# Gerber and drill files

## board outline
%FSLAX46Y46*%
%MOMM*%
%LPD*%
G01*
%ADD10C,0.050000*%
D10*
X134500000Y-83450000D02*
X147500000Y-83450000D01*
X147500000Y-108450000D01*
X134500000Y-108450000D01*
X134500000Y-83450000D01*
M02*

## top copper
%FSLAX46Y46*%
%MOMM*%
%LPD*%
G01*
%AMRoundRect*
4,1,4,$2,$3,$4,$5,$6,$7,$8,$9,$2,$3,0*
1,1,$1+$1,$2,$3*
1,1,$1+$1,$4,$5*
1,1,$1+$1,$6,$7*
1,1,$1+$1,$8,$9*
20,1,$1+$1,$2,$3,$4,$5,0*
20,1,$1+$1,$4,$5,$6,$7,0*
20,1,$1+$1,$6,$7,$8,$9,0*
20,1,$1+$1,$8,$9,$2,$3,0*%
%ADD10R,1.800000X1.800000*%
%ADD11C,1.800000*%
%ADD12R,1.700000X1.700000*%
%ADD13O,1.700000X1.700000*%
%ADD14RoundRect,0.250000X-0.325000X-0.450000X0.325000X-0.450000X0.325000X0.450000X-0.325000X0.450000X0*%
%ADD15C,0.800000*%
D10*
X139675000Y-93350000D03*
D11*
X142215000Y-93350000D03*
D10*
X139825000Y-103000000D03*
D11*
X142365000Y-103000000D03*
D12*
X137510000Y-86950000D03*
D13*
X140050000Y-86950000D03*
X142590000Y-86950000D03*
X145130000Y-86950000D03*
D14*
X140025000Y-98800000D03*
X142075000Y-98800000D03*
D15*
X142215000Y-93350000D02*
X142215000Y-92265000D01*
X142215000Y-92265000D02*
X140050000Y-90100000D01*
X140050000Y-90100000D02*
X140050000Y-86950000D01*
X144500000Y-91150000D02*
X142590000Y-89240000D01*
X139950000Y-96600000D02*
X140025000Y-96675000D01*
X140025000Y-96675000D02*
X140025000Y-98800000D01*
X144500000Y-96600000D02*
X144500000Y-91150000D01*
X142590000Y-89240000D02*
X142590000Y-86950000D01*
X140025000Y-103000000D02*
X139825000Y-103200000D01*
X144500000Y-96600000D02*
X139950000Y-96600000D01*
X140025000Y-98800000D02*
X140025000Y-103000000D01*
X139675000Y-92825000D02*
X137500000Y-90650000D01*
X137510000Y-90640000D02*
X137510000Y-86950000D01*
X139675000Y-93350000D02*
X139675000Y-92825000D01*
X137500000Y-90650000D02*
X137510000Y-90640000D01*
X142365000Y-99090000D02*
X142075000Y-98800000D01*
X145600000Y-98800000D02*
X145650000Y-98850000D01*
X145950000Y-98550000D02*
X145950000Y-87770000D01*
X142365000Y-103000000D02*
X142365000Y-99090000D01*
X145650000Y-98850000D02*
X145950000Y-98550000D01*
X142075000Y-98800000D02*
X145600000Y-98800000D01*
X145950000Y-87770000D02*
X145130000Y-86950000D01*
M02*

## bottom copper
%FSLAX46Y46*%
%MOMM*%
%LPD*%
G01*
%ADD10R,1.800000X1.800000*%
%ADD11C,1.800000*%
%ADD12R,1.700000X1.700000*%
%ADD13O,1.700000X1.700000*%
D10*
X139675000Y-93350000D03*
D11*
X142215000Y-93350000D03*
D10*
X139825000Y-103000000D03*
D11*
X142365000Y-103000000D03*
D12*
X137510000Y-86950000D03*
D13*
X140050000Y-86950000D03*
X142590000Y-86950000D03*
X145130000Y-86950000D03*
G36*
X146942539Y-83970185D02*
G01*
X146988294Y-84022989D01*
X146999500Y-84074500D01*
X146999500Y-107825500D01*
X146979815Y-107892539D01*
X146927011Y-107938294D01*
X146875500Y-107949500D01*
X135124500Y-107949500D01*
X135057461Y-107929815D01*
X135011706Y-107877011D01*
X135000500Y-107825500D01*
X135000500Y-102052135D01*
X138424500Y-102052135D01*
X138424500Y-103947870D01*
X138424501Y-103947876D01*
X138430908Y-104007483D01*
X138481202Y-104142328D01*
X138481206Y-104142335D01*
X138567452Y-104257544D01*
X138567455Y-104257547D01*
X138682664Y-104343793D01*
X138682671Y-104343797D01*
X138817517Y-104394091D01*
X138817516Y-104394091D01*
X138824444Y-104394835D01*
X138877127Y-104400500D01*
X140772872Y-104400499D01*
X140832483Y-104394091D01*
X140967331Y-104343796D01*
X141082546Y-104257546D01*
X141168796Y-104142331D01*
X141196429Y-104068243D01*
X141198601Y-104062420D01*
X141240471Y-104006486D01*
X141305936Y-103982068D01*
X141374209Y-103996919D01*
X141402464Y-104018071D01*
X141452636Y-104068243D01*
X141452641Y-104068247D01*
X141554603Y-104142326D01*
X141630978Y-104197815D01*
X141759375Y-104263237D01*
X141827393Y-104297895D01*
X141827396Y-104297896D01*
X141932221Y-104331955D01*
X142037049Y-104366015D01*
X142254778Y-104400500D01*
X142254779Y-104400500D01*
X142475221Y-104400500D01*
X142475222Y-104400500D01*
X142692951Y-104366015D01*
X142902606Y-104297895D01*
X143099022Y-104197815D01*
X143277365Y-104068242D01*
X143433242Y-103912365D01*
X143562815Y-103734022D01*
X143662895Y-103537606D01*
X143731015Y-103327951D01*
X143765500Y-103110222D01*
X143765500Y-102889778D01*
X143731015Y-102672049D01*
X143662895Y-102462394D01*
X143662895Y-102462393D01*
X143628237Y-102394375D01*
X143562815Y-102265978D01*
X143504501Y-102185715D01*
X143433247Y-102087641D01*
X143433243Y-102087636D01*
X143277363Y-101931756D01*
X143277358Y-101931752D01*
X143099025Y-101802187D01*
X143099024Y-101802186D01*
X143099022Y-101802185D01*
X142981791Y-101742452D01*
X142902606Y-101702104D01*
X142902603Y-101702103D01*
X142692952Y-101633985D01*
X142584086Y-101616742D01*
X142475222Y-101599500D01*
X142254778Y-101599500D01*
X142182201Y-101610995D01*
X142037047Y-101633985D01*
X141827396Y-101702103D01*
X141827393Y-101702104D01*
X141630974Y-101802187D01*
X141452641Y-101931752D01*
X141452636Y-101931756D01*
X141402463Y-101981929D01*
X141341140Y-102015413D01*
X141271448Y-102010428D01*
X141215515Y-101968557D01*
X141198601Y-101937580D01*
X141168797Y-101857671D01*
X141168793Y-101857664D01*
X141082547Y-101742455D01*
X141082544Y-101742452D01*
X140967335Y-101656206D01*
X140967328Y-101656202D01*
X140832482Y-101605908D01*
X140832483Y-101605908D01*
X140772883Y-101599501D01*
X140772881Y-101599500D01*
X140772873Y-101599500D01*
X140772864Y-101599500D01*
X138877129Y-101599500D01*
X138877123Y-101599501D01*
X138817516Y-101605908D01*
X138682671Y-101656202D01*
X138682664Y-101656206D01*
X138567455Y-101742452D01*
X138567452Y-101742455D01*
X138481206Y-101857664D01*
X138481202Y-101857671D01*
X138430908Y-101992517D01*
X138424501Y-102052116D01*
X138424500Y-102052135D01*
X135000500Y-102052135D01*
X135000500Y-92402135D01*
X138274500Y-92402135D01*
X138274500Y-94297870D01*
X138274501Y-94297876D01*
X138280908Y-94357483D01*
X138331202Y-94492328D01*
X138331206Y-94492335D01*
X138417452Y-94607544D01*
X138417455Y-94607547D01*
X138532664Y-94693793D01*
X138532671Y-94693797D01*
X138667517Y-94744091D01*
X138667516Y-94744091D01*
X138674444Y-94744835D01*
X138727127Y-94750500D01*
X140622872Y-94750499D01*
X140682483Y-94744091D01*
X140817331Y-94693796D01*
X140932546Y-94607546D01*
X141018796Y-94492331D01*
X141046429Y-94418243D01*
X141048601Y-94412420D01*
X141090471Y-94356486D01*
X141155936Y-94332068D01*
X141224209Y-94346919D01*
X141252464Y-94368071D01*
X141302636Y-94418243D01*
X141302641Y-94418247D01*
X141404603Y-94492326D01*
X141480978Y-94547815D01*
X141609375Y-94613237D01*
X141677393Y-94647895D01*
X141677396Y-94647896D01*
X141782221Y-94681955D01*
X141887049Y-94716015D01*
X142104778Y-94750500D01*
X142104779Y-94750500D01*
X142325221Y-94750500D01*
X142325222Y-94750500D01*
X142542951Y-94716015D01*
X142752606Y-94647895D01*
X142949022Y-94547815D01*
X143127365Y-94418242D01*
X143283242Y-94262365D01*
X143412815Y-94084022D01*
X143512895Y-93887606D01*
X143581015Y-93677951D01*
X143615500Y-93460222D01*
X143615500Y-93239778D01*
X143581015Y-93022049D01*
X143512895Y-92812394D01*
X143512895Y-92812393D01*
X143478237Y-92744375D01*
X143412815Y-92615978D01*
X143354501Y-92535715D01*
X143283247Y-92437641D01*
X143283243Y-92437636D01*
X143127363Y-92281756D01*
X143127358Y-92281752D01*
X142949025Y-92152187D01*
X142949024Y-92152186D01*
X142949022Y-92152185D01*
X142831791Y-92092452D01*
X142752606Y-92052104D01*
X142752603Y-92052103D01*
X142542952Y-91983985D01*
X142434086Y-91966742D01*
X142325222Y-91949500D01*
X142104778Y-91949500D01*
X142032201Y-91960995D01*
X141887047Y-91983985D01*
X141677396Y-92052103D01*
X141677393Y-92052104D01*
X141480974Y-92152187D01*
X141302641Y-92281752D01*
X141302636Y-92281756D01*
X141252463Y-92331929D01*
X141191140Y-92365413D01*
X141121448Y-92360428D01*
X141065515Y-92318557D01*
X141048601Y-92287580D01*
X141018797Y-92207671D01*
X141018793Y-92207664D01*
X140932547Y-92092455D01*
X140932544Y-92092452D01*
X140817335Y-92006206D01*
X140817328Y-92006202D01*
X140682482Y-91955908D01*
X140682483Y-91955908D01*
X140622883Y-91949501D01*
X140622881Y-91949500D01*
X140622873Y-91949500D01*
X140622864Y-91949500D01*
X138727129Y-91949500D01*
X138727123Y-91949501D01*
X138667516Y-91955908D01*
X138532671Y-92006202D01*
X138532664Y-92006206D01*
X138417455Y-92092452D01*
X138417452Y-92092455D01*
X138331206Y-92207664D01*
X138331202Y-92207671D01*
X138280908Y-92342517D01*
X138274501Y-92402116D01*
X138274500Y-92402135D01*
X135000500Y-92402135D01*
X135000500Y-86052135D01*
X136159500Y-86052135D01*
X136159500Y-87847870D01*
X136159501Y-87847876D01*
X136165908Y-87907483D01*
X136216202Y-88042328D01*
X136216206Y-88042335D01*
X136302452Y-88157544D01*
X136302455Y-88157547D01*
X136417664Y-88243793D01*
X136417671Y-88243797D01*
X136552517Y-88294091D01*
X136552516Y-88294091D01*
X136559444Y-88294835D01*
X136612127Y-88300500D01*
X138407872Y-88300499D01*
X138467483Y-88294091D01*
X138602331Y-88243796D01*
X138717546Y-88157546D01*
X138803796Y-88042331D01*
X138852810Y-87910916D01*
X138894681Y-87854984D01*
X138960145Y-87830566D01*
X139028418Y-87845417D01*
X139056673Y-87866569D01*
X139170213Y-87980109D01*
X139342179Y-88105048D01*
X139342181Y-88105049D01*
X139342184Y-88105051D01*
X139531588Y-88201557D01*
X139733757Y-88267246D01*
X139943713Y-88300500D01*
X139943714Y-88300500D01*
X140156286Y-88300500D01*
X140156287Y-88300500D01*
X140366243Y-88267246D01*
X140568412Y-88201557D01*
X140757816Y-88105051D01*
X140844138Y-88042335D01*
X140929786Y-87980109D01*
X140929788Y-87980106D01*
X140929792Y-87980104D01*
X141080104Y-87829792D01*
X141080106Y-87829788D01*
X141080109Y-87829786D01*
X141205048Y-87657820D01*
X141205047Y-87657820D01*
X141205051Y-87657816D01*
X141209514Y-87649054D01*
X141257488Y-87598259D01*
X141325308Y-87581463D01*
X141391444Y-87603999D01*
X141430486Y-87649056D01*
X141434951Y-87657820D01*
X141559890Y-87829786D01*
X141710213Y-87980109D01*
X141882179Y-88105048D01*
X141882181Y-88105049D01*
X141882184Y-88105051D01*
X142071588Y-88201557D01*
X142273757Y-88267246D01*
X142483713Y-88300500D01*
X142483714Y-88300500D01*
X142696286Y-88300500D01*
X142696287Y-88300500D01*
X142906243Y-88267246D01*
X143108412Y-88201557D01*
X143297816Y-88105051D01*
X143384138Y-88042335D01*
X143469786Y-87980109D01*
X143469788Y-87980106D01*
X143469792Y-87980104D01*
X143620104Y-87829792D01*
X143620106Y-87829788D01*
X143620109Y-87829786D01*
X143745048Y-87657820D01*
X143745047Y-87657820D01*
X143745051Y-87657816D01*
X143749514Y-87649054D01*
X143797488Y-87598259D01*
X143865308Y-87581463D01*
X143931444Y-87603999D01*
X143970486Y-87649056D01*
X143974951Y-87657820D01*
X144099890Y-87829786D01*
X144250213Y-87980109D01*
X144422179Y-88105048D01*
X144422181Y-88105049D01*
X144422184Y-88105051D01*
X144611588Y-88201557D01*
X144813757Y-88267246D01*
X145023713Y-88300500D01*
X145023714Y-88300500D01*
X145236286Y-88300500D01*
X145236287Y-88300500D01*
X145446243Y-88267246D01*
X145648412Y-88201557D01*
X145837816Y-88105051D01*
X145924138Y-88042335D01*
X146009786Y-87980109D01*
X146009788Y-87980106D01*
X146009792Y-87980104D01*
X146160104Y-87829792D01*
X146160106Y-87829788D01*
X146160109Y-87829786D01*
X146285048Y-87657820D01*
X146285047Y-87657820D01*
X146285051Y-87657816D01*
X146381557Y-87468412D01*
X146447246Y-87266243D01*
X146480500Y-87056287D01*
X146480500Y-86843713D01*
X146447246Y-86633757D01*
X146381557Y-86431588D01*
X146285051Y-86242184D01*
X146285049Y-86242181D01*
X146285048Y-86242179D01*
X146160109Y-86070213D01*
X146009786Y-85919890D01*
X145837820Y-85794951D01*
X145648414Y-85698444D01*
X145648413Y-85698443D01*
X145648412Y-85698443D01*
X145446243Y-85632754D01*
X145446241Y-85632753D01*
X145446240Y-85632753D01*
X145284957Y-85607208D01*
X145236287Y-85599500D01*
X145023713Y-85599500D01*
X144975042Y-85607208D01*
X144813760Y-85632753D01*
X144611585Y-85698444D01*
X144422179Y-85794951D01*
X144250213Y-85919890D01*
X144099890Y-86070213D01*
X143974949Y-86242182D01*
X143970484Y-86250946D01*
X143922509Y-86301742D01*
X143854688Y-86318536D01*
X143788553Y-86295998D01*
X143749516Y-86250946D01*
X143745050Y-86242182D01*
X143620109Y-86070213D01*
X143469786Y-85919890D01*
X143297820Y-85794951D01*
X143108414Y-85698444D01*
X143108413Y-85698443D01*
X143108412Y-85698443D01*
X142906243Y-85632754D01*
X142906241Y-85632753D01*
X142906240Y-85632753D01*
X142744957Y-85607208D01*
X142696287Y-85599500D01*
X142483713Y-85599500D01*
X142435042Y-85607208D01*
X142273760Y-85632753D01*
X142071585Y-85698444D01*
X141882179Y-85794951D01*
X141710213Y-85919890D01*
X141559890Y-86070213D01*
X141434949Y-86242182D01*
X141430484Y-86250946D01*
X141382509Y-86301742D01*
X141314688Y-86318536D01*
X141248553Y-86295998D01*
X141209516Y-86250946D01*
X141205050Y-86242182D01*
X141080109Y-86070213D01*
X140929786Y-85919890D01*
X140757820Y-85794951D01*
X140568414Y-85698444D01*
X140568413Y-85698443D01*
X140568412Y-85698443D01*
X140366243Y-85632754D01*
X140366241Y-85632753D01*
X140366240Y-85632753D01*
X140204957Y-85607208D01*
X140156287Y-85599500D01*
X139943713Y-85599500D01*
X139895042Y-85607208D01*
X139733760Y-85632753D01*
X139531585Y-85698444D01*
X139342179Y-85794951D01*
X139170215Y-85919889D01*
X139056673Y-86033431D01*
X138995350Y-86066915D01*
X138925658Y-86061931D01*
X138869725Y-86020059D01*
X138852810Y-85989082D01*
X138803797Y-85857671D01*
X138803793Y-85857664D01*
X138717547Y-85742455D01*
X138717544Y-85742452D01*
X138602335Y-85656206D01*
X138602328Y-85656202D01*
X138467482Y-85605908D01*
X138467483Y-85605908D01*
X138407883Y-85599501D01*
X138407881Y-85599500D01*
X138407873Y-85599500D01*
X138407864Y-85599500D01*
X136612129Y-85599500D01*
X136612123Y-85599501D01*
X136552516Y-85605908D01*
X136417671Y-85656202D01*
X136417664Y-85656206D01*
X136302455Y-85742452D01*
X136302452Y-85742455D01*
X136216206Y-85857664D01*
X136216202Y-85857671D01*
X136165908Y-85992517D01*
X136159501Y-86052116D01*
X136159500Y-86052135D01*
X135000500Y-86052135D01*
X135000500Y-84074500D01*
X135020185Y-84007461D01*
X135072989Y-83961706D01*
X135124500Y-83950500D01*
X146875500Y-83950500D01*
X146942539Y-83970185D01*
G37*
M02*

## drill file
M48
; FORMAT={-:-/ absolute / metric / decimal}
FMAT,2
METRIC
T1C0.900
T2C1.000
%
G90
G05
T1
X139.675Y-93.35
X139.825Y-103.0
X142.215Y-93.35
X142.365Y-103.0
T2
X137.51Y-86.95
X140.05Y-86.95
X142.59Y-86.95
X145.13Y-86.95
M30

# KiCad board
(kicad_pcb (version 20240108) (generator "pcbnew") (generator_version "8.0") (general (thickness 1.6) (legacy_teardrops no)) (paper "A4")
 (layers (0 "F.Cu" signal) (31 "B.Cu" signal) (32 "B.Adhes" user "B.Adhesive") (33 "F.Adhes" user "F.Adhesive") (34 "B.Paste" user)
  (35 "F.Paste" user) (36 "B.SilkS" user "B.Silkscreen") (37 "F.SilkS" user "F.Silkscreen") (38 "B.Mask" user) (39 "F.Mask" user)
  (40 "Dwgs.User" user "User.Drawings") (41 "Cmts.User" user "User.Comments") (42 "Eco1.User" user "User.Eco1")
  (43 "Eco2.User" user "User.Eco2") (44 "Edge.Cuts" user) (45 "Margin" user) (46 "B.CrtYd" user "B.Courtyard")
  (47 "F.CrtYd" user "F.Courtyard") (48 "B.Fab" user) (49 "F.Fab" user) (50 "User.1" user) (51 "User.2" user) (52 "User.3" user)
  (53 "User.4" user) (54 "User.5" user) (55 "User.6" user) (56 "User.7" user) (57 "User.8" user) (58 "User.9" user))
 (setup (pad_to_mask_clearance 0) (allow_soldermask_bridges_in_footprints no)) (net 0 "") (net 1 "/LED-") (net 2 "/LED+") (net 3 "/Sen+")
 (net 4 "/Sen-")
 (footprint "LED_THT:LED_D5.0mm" (layer "F.Cu") (at 139.675 93.35)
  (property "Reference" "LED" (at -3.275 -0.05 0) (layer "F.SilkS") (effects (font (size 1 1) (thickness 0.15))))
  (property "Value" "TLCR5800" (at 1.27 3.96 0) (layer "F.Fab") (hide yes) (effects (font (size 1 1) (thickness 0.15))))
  (pad "1" thru_hole rect (at 0 0) (size 1.8 1.8) (drill 0.9) (layers "*.Cu" "*.Mask") (remove_unused_layers no) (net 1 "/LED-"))
  (pad "2" thru_hole circle (at 2.54 0) (size 1.8 1.8) (drill 0.9) (layers "*.Cu" "*.Mask") (remove_unused_layers no) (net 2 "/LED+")))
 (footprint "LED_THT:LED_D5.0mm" (layer "F.Cu") (at 139.825 103)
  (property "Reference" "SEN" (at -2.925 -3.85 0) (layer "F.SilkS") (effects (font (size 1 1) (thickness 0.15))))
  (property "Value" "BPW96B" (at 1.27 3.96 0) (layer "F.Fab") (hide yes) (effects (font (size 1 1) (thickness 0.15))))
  (pad "1" thru_hole rect (at 0 0) (size 1.8 1.8) (drill 0.9) (layers "*.Cu" "*.Mask") (remove_unused_layers no) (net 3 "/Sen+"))
  (pad "2" thru_hole circle (at 2.54 0) (size 1.8 1.8) (drill 0.9) (layers "*.Cu" "*.Mask") (remove_unused_layers no) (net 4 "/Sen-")))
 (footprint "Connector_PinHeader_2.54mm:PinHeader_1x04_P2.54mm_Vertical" (layer "F.Cu") (at 137.51 86.95 90)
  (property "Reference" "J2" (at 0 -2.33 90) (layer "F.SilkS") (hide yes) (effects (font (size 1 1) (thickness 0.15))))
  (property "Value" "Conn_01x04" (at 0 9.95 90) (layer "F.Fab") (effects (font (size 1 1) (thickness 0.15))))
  (pad "1" thru_hole rect (at 0 0 90) (size 1.7 1.7) (drill 1) (layers "*.Cu" "*.Mask") (remove_unused_layers no) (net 1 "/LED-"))
  (pad "2" thru_hole oval (at 0 2.54 90) (size 1.7 1.7) (drill 1) (layers "*.Cu" "*.Mask") (remove_unused_layers no) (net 2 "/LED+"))
  (pad "3" thru_hole oval (at 0 5.08 90) (size 1.7 1.7) (drill 1) (layers "*.Cu" "*.Mask") (remove_unused_layers no) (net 3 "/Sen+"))
  (pad "4" thru_hole oval (at 0 7.62 90) (size 1.7 1.7) (drill 1) (layers "*.Cu" "*.Mask") (remove_unused_layers no) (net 4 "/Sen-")))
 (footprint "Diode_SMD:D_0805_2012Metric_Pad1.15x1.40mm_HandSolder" (layer "F.Cu") (at 141.05 98.8)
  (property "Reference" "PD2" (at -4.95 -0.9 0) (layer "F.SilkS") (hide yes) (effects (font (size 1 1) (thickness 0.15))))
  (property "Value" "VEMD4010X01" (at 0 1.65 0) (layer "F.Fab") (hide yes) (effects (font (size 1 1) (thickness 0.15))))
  (pad "1" smd roundrect (at -1.025 0) (size 1.15 1.4) (layers "F.Cu" "F.Paste" "F.Mask") (roundrect_rratio 0.217391) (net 3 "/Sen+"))
  (pad "2" smd roundrect (at 1.025 0) (size 1.15 1.4) (layers "F.Cu" "F.Paste" "F.Mask") (roundrect_rratio 0.217391) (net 4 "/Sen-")))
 (gr_rect (start 134.5 83.45) (end 147.5 108.45) (stroke (width 0.05) (type default)) (fill none) (layer "Edge.Cuts"))
 (segment (start 142.215 93.35) (end 142.215 92.265) (width 0.8) (layer "F.Cu") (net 2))
 (segment (start 142.215 92.265) (end 140.05 90.1) (width 0.8) (layer "F.Cu") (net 2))
 (segment (start 140.05 90.1) (end 140.05 86.95) (width 0.8) (layer "F.Cu") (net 2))
 (segment (start 144.5 91.15) (end 142.59 89.24) (width 0.8) (layer "F.Cu") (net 3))
 (segment (start 139.95 96.6) (end 140.025 96.675) (width 0.8) (layer "F.Cu") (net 3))
 (segment (start 140.025 96.675) (end 140.025 98.8) (width 0.8) (layer "F.Cu") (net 3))
 (segment (start 144.5 96.6) (end 144.5 91.15) (width 0.8) (layer "F.Cu") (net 3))
 (segment (start 142.59 89.24) (end 142.59 86.95) (width 0.8) (layer "F.Cu") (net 3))
 (segment (start 140.025 103) (end 139.825 103.2) (width 0.8) (layer "F.Cu") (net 3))
 (segment (start 144.5 96.6) (end 139.95 96.6) (width 0.8) (layer "F.Cu") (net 3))
 (segment (start 140.025 98.8) (end 140.025 103) (width 0.8) (layer "F.Cu") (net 3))
 (segment (start 139.675 92.825) (end 137.5 90.65) (width 0.8) (layer "F.Cu") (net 1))
 (segment (start 137.51 90.64) (end 137.51 86.95) (width 0.8) (layer "F.Cu") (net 1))
 (segment (start 139.675 93.35) (end 139.675 92.825) (width 0.8) (layer "F.Cu") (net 1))
 (segment (start 137.5 90.65) (end 137.51 90.64) (width 0.8) (layer "F.Cu") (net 1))
 (segment (start 142.365 99.09) (end 142.075 98.8) (width 0.8) (layer "F.Cu") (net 4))
 (segment (start 145.6 98.8) (end 145.65 98.85) (width 0.8) (layer "F.Cu") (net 4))
 (segment (start 145.95 98.55) (end 145.95 87.77) (width 0.8) (layer "F.Cu") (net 4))
 (segment (start 142.365 103) (end 142.365 99.09) (width 0.8) (layer "F.Cu") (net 4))
 (segment (start 145.65 98.85) (end 145.95 98.55) (width 0.8) (layer "F.Cu") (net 4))
 (segment (start 142.075 98.8) (end 145.6 98.8) (width 0.8) (layer "F.Cu") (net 4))
 (segment (start 145.95 87.77) (end 145.13 86.95) (width 0.8) (layer "F.Cu") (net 4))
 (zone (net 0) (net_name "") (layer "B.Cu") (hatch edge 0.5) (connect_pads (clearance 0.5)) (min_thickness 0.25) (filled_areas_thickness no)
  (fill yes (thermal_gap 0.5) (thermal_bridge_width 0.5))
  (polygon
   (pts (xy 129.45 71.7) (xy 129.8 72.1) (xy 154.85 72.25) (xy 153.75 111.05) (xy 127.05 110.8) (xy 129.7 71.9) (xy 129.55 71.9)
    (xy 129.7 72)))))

